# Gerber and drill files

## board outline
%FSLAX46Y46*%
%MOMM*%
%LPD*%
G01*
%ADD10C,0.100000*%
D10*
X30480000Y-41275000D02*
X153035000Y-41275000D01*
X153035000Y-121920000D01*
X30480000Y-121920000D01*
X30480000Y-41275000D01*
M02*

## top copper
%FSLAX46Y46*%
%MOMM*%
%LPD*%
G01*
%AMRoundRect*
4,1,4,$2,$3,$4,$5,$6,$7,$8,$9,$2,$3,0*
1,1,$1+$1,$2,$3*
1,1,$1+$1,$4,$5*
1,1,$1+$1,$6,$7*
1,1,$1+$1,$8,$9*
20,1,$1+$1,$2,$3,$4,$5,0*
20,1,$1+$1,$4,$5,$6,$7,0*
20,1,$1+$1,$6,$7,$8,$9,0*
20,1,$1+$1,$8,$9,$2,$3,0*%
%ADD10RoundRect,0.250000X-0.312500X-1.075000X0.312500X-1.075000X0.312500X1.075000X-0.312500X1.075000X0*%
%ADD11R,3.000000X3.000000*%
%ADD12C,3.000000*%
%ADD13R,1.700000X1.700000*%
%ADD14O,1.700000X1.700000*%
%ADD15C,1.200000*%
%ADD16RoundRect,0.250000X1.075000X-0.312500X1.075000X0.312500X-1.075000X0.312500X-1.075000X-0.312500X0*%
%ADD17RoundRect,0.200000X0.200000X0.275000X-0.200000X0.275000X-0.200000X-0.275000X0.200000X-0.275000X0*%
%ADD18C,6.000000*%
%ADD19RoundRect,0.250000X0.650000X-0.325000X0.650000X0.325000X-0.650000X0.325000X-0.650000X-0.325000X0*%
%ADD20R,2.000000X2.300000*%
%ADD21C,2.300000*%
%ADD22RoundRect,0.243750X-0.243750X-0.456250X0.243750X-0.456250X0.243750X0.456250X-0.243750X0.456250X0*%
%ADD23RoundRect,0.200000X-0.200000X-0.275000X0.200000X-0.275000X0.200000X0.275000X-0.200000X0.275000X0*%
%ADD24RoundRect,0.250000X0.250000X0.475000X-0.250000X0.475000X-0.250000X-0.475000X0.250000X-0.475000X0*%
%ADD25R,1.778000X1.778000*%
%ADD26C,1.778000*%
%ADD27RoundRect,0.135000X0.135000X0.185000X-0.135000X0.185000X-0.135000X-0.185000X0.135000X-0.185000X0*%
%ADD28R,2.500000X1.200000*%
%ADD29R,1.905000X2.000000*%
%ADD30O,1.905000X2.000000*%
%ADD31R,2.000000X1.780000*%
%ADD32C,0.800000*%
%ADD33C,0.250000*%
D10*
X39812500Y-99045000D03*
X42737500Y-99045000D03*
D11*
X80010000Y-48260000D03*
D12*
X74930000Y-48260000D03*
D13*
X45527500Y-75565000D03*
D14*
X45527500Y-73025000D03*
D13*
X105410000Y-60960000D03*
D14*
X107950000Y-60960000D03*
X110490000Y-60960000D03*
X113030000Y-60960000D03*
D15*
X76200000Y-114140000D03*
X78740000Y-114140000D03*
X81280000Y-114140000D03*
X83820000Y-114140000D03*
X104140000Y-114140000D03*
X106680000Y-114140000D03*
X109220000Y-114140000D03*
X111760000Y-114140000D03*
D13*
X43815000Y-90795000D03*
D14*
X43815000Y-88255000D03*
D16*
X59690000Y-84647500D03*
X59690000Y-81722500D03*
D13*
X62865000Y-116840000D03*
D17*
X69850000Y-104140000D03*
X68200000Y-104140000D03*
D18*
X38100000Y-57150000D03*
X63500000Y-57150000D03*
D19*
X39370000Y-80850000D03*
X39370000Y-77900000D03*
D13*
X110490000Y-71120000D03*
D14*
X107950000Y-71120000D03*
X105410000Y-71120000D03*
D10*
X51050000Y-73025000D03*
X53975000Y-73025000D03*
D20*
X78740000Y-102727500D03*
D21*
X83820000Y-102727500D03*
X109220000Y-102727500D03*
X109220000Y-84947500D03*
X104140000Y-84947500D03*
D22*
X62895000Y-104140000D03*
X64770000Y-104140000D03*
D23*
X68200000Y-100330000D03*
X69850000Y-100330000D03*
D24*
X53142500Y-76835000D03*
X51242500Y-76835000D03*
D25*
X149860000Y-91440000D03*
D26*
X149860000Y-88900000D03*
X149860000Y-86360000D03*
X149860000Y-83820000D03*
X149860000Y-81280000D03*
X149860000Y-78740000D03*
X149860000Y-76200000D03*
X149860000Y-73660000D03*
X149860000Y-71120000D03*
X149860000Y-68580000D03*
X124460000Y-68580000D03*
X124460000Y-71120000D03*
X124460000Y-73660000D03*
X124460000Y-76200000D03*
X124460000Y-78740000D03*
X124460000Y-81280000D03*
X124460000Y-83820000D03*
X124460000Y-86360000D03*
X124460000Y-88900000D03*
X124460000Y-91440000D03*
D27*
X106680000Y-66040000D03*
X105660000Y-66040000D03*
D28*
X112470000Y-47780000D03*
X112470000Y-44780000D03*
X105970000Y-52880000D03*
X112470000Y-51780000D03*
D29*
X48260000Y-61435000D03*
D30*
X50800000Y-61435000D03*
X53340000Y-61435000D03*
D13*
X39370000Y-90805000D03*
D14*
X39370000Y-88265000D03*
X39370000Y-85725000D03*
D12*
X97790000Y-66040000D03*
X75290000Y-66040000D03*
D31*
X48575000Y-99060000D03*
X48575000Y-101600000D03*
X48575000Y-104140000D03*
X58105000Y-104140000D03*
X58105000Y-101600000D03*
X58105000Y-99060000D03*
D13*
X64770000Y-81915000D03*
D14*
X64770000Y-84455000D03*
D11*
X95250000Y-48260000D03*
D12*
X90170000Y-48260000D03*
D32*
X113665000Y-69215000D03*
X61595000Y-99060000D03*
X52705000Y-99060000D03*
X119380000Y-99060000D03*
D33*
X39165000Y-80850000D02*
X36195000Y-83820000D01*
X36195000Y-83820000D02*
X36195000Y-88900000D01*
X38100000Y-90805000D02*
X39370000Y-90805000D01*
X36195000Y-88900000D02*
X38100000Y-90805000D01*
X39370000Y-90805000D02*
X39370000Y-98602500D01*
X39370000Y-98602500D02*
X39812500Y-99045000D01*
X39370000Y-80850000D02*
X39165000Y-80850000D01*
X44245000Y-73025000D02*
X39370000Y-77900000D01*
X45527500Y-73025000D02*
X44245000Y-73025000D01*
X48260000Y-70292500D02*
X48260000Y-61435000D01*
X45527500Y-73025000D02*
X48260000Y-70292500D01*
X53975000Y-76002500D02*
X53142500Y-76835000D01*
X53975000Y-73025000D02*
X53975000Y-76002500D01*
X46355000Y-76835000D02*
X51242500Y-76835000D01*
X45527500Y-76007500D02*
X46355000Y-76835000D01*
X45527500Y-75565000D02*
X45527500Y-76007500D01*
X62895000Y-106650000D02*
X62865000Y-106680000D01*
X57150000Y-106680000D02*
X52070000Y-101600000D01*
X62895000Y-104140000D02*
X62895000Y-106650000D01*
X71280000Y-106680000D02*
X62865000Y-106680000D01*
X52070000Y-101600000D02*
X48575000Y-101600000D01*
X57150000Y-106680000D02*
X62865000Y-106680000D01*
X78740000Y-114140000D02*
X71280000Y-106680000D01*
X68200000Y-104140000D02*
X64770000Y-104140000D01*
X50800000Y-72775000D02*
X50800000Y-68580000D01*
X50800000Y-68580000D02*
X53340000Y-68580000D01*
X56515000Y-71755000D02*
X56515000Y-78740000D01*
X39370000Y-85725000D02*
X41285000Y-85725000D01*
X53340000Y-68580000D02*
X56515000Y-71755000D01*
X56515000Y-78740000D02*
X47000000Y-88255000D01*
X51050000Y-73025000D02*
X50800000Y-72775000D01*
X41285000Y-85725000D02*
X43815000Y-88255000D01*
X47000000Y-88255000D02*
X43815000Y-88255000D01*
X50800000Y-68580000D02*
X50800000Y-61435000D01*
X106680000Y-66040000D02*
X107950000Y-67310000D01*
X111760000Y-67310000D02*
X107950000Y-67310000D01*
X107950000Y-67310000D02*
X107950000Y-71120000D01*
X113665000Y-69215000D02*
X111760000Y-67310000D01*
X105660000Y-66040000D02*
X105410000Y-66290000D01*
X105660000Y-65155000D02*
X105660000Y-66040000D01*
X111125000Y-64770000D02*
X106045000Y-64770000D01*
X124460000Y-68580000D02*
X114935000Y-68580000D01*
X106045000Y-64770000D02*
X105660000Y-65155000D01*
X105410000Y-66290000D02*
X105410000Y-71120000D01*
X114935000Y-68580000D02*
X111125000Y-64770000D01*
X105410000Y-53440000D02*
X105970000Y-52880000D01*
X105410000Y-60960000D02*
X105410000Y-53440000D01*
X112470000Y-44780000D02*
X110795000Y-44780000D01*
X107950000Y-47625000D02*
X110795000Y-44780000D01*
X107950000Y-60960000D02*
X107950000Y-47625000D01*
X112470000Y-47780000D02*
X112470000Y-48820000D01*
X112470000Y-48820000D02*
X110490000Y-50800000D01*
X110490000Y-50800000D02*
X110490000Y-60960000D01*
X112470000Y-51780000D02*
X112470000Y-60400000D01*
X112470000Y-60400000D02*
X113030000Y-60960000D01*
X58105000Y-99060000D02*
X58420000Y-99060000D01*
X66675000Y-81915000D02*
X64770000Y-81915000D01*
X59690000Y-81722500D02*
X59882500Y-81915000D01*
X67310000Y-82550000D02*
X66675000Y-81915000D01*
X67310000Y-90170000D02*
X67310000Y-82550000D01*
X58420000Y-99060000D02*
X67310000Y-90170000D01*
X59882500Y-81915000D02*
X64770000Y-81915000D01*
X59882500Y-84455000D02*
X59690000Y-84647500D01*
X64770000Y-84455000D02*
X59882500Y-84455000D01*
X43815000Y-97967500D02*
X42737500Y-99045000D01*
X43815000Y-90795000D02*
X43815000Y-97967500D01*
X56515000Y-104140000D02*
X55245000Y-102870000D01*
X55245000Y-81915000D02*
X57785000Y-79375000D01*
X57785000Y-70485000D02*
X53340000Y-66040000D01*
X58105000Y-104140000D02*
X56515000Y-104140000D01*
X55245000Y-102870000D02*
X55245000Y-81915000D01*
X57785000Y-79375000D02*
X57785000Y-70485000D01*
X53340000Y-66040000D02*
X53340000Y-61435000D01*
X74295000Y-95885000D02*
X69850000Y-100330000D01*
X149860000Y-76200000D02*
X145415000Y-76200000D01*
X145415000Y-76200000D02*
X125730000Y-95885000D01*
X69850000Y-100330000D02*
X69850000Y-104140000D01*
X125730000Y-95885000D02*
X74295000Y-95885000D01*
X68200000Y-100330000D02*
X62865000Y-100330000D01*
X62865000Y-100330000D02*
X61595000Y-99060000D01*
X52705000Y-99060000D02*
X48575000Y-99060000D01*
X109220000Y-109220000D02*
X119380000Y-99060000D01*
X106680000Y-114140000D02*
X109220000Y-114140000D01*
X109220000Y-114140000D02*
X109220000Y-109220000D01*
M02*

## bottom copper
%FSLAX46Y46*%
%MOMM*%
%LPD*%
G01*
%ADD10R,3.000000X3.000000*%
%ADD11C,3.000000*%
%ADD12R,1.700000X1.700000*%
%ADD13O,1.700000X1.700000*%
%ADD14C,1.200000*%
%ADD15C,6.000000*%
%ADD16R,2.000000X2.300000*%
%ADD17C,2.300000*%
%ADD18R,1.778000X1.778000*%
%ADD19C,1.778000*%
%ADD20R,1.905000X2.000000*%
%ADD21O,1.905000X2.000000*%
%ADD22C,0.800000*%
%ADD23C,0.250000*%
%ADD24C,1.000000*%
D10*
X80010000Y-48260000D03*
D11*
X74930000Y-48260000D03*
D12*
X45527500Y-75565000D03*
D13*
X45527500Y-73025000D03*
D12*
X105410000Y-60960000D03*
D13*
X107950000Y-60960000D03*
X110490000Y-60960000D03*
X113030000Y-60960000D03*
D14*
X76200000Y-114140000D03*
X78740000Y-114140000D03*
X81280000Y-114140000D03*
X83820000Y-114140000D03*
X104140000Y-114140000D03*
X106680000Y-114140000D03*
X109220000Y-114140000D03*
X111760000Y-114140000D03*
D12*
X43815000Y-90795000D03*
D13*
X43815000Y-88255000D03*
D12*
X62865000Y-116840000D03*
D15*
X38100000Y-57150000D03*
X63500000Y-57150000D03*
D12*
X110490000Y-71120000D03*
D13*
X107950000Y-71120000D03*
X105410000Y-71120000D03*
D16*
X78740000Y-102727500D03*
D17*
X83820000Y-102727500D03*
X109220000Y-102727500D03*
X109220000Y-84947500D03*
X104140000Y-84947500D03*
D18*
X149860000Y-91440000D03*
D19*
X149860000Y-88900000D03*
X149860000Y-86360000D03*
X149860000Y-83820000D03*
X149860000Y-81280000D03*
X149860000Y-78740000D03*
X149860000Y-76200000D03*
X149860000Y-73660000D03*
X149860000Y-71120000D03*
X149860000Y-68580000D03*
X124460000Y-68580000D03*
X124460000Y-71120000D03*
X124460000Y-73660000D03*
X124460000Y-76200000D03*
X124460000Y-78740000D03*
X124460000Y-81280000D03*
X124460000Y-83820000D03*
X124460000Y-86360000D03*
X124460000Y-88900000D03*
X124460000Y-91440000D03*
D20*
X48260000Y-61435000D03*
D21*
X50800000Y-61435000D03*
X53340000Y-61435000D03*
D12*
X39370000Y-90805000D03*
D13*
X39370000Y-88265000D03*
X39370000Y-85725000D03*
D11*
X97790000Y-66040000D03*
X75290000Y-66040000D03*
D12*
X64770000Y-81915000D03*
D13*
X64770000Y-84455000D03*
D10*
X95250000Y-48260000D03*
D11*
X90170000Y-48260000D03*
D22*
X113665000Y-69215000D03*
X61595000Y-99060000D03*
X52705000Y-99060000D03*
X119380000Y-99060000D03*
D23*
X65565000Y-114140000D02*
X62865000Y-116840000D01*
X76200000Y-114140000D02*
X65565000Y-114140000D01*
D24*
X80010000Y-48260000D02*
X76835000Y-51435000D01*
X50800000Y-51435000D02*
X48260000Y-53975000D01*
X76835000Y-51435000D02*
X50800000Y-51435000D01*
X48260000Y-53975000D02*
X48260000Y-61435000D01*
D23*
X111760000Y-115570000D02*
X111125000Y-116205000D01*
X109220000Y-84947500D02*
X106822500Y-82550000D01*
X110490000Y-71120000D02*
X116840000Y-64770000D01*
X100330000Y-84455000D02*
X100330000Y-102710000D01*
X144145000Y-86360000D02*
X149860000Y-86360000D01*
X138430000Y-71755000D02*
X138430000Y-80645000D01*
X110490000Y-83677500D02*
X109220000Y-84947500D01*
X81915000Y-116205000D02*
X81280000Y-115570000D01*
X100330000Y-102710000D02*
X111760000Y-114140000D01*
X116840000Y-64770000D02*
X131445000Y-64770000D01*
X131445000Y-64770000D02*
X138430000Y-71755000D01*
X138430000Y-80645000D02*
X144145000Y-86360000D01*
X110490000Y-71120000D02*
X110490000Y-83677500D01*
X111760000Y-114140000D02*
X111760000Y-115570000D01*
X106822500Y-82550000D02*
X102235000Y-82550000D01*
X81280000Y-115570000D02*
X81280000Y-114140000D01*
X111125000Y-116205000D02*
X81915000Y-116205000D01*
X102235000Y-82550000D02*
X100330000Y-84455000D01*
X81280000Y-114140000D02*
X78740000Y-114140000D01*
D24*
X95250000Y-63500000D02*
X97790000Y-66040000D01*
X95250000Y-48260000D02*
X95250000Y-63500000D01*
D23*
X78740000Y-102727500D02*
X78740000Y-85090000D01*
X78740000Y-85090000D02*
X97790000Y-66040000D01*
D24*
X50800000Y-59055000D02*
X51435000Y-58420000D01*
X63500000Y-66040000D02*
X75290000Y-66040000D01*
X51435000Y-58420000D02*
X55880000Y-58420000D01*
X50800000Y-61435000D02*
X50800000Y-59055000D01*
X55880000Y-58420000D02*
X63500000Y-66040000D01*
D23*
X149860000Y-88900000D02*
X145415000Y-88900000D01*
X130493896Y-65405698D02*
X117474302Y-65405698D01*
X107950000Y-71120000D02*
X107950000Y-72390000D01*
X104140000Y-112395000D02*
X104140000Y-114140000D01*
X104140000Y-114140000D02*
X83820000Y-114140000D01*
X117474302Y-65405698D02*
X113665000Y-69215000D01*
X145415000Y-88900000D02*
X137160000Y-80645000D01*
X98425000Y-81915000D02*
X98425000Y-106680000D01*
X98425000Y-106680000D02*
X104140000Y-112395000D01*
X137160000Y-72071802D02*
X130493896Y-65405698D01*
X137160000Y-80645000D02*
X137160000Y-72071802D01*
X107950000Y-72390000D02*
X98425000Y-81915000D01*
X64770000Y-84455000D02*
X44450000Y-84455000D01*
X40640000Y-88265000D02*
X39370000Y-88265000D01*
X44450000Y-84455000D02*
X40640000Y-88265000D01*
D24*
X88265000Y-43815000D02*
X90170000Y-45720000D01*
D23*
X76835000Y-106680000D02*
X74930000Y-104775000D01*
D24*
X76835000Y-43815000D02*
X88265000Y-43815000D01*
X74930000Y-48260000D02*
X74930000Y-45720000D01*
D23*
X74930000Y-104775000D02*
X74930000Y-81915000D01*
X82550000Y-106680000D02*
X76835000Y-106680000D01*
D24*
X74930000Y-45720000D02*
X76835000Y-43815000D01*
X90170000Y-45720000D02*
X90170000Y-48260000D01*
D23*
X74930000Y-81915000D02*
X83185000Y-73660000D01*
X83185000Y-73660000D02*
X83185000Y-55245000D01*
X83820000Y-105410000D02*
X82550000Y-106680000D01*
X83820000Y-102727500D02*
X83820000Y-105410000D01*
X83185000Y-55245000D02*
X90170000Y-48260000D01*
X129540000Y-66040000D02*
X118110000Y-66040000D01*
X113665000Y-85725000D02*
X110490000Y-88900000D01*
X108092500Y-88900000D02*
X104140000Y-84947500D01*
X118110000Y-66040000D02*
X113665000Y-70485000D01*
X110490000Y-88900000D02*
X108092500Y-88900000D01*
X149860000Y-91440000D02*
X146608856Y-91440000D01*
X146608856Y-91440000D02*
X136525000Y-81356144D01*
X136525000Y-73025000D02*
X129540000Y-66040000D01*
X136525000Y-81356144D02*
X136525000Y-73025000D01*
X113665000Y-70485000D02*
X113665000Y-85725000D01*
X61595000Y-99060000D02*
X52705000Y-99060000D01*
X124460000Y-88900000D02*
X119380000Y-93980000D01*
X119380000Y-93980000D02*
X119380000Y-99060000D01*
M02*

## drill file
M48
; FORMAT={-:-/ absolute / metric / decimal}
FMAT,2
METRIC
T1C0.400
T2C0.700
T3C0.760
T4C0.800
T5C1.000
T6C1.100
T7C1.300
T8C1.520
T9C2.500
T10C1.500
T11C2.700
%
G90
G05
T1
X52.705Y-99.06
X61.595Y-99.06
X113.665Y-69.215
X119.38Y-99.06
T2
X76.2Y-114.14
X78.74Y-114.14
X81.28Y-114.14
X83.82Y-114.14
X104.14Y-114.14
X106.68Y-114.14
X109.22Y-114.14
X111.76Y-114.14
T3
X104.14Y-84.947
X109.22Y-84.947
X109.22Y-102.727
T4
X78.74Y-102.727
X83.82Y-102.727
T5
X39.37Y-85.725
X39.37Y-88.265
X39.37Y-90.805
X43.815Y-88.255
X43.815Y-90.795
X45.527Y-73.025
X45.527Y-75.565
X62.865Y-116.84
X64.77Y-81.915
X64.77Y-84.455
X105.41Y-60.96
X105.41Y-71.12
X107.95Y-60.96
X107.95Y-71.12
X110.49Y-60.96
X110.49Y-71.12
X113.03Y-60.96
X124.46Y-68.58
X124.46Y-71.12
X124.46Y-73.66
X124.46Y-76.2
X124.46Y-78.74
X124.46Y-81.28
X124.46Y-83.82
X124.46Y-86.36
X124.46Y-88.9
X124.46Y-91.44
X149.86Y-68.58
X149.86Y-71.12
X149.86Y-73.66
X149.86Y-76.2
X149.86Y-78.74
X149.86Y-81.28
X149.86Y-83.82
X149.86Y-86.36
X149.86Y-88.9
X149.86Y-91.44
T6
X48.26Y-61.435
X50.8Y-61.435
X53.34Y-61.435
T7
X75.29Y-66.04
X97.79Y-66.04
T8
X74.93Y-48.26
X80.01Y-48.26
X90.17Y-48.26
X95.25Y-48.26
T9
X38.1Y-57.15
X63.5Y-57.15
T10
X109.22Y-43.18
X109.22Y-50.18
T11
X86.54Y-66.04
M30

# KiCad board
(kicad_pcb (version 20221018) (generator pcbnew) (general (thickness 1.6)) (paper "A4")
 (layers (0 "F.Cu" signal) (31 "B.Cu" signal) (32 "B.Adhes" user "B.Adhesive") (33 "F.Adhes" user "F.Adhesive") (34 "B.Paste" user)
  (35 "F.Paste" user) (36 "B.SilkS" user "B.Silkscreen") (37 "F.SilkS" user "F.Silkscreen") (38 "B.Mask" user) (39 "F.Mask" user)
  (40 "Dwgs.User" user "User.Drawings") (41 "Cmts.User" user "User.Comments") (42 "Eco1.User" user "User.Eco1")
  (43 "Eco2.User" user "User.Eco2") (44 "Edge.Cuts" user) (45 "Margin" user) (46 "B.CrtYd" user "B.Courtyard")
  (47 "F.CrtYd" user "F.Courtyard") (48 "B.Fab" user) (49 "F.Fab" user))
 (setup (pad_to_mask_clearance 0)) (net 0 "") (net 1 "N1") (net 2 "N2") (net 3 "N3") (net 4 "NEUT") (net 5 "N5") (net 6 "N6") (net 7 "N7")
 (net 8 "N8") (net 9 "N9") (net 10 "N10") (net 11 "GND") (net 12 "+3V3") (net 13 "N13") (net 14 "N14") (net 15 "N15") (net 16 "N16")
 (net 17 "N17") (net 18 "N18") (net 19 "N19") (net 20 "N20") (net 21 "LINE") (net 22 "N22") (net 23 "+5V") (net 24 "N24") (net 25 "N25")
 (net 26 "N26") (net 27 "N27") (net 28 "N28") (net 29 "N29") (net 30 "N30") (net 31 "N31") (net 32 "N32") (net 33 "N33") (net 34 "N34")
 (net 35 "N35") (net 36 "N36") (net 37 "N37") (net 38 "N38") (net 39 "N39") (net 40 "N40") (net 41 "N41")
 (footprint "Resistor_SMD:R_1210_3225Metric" (layer "F.Cu") (at 41.275 99.045)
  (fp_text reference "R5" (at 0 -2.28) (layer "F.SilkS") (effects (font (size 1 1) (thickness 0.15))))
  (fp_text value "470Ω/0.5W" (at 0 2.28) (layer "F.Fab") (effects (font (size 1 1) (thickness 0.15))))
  (pad "1" smd roundrect (at -1.4625 0) (size 1.125 2.65) (layers "F.Cu" "F.Paste" "F.Mask") (roundrect_rratio 0.2222222222) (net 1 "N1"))
  (pad "2" smd roundrect (at 1.4625 0) (size 1.125 2.65) (layers "F.Cu" "F.Paste" "F.Mask") (roundrect_rratio 0.2222222222) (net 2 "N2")))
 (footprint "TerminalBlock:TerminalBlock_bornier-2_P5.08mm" (layer "F.Cu") (at 80.01 48.26 180)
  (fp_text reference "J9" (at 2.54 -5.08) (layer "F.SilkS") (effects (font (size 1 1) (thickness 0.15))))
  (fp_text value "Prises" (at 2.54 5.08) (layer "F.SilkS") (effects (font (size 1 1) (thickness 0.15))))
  (pad "1" thru_hole rect (at 0 0 180) (size 3 3) (drill 1.52) (layers "*.Cu" "*.Mask") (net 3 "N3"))
  (pad "2" thru_hole circle (at 5.08 0 180) (size 3 3) (drill 1.52) (layers "*.Cu" "*.Mask") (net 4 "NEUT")))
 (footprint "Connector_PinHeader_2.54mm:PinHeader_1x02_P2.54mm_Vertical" (layer "F.Cu") (at 45.5275 75.565 180)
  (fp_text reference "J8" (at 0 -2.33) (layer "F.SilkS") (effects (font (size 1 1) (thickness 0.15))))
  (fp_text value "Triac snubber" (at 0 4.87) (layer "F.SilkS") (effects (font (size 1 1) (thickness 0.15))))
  (pad "1" thru_hole rect (at 0 0 180) (size 1.7 1.7) (drill 1) (layers "*.Cu" "*.Mask") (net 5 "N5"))
  (pad "2" thru_hole oval (at 0 2.54 180) (size 1.7 1.7) (drill 1) (layers "*.Cu" "*.Mask") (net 3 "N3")))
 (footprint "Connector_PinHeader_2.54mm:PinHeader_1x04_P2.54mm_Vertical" (layer "F.Cu") (at 105.41 60.96 90)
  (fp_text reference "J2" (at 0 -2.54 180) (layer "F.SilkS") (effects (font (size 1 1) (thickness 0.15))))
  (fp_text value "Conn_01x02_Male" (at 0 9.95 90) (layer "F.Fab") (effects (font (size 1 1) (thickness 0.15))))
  (pad "1" thru_hole rect (at 0 0 90) (size 1.7 1.7) (drill 1) (layers "*.Cu" "*.Mask") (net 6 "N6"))
  (pad "2" thru_hole oval (at 0 2.54 90) (size 1.7 1.7) (drill 1) (layers "*.Cu" "*.Mask") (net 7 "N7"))
  (pad "3" thru_hole oval (at 0 5.08 90) (size 1.7 1.7) (drill 1) (layers "*.Cu" "*.Mask") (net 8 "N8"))
  (pad "4" thru_hole oval (at 0 7.62 90) (size 1.7 1.7) (drill 1) (layers "*.Cu" "*.Mask") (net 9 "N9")))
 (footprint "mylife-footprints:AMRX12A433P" (layer "F.Cu") (at 93.98 116.84)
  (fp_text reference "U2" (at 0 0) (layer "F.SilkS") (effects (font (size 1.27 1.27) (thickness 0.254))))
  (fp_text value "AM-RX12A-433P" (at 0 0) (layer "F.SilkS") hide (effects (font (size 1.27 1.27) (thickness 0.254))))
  (pad "1" thru_hole circle (at -17.78 -2.7) (size 1.2 1.2) (drill 0.7) (layers "*.Cu" "*.Mask") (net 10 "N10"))
  (pad "2" thru_hole circle (at -15.24 -2.7) (size 1.2 1.2) (drill 0.7) (layers "*.Cu" "*.Mask") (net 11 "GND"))
  (pad "3" thru_hole circle (at -12.7 -2.7) (size 1.2 1.2) (drill 0.7) (layers "*.Cu" "*.Mask") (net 11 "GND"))
  (pad "4" thru_hole circle (at -10.16 -2.7) (size 1.2 1.2) (drill 0.7) (layers "*.Cu" "*.Mask") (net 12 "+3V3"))
  (pad "5" thru_hole circle (at 10.16 -2.7) (size 1.2 1.2) (drill 0.7) (layers "*.Cu" "*.Mask") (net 12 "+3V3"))
  (pad "6" thru_hole circle (at 12.7 -2.7) (size 1.2 1.2) (drill 0.7) (layers "*.Cu" "*.Mask") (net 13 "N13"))
  (pad "7" thru_hole circle (at 15.24 -2.7) (size 1.2 1.2) (drill 0.7) (layers "*.Cu" "*.Mask") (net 13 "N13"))
  (pad "8" thru_hole circle (at 17.78 -2.7) (size 1.2 1.2) (drill 0.7) (layers "*.Cu" "*.Mask") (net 11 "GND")))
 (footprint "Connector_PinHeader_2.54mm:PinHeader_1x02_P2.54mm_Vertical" (layer "F.Cu") (at 43.815 90.795 180)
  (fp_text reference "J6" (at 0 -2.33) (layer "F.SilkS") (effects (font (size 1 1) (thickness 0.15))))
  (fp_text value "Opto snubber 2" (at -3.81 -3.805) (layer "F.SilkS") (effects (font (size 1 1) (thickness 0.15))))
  (pad "1" thru_hole rect (at 0 0 180) (size 1.7 1.7) (drill 1) (layers "*.Cu" "*.Mask") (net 2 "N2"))
  (pad "2" thru_hole oval (at 0 2.54 180) (size 1.7 1.7) (drill 1) (layers "*.Cu" "*.Mask") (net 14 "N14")))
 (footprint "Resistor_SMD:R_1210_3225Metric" (layer "F.Cu") (at 59.69 83.185 90)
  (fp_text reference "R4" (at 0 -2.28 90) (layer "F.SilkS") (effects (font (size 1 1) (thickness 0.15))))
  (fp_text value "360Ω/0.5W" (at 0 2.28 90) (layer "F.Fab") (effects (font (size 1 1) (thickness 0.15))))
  (pad "1" smd roundrect (at -1.4625 0 90) (size 1.125 2.65) (layers "F.Cu" "F.Paste" "F.Mask") (roundrect_rratio 0.2222222222)
   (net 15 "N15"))
  (pad "2" smd roundrect (at 1.4625 0 90) (size 1.125 2.65) (layers "F.Cu" "F.Paste" "F.Mask") (roundrect_rratio 0.2222222222)
   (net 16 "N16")))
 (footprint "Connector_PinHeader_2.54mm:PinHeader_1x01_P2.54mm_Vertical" (layer "F.Cu") (at 62.865 116.84)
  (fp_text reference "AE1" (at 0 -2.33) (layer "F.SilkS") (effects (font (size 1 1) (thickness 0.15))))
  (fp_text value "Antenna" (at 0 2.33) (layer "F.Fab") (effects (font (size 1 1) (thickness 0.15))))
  (pad "1" thru_hole rect (at 0 0) (size 1.7 1.7) (drill 1) (layers "*.Cu" "*.Mask") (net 10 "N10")))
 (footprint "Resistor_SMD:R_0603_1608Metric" (layer "F.Cu") (at 69.025 104.14 180)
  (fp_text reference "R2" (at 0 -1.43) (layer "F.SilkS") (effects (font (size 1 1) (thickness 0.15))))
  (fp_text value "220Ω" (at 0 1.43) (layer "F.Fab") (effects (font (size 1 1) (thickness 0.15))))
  (pad "1" smd roundrect (at -0.825 0 180) (size 0.8 0.95) (layers "F.Cu" "F.Paste" "F.Mask") (roundrect_rratio 0.25) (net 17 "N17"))
  (pad "2" smd roundrect (at 0.825 0 180) (size 0.8 0.95) (layers "F.Cu" "F.Paste" "F.Mask") (roundrect_rratio 0.25) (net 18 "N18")))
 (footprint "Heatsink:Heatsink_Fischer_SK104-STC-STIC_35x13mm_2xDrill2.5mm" (layer "F.Cu") (at 50.8 57.15)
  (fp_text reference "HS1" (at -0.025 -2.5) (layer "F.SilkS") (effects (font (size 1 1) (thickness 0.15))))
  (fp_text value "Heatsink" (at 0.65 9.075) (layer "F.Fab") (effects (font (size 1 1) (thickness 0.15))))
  (pad "1" thru_hole circle (at -12.7 0 180) (size 6 6) (drill 2.5) (layers "*.Cu" "*.Mask"))
  (pad "1" thru_hole circle (at 12.7 0) (size 6 6) (drill 2.5) (layers "*.Cu" "*.Mask")))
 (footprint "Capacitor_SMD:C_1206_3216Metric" (layer "F.Cu") (at 39.37 79.375 90)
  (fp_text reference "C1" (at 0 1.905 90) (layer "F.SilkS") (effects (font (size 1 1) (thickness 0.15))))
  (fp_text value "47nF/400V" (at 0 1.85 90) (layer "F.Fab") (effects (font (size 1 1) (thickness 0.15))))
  (pad "1" smd roundrect (at -1.475 0 90) (size 1.15 1.8) (layers "F.Cu" "F.Paste" "F.Mask") (roundrect_rratio 0.2173913043) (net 1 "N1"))
  (pad "2" smd roundrect (at 1.475 0 90) (size 1.15 1.8) (layers "F.Cu" "F.Paste" "F.Mask") (roundrect_rratio 0.2173913043) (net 3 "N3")))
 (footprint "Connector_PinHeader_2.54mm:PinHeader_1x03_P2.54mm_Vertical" (layer "F.Cu") (at 110.49 71.12 -90)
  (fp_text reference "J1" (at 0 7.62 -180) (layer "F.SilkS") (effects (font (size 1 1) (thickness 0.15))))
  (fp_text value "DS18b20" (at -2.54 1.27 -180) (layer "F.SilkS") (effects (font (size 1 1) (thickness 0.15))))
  (pad "1" thru_hole rect (at 0 0 270) (size 1.7 1.7) (drill 1) (layers "*.Cu" "*.Mask") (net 11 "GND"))
  (pad "2" thru_hole oval (at 0 2.54 270) (size 1.7 1.7) (drill 1) (layers "*.Cu" "*.Mask") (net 12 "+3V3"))
  (pad "3" thru_hole oval (at 0 5.08 270) (size 1.7 1.7) (drill 1) (layers "*.Cu" "*.Mask") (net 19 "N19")))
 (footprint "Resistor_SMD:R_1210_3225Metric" (layer "F.Cu") (at 52.5125 73.025)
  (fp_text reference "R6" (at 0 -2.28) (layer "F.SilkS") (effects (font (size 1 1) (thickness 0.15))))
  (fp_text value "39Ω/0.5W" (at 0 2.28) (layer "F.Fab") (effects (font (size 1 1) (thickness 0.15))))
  (pad "1" smd roundrect (at -1.4625 0) (size 1.125 2.65) (layers "F.Cu" "F.Paste" "F.Mask") (roundrect_rratio 0.2222222222) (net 14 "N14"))
  (pad "2" smd roundrect (at 1.4625 0) (size 1.125 2.65) (layers "F.Cu" "F.Paste" "F.Mask") (roundrect_rratio 0.2222222222) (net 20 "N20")))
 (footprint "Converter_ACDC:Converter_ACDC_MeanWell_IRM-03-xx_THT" (layer "F.Cu") (at 78.74 102.7275 90)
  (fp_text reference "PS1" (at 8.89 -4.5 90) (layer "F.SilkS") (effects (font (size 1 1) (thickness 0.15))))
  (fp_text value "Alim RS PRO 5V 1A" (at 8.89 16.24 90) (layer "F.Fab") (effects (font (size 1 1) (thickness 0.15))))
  (pad "1" thru_hole rect (at 0 0 90) (size 2.3 2) (drill 0.8) (layers "*.Cu" "*.Mask") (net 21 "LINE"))
  (pad "3" thru_hole circle (at 0 5.08 90) (size 2.3 2.3) (drill 0.8) (layers "*.Cu" "*.Mask") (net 4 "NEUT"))
  (pad "5" thru_hole circle (at 0 30.48 90) (size 2.3 2.3) (drill 0.76) (layers "*.Cu" "*.Mask") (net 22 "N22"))
  (pad "14" thru_hole circle (at 17.78 30.48 90) (size 2.3 2.3) (drill 0.76) (layers "*.Cu" "*.Mask") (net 11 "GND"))
  (pad "16" thru_hole circle (at 17.78 25.4 90) (size 2.3 2.3) (drill 0.76) (layers "*.Cu" "*.Mask") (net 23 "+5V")))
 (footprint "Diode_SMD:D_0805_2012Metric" (layer "F.Cu") (at 63.8325 104.14)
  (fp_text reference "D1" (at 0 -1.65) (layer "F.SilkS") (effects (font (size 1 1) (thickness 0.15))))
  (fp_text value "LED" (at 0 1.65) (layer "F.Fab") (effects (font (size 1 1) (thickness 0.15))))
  (pad "1" smd roundrect (at -0.9375 0) (size 0.975 1.4) (layers "F.Cu" "F.Paste" "F.Mask") (roundrect_rratio 0.25) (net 11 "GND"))
  (pad "2" smd roundrect (at 0.9375 0) (size 0.975 1.4) (layers "F.Cu" "F.Paste" "F.Mask") (roundrect_rratio 0.25) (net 18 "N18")))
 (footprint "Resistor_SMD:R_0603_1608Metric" (layer "F.Cu") (at 69.025 100.33)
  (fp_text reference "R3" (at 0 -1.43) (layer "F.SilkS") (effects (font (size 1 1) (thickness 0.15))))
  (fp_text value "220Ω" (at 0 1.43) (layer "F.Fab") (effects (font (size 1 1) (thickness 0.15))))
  (pad "1" smd roundrect (at -0.825 0) (size 0.8 0.95) (layers "F.Cu" "F.Paste" "F.Mask") (roundrect_rratio 0.25) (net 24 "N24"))
  (pad "2" smd roundrect (at 0.825 0) (size 0.8 0.95) (layers "F.Cu" "F.Paste" "F.Mask") (roundrect_rratio 0.25) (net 17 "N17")))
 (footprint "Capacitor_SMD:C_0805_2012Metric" (layer "F.Cu") (at 52.1925 76.835 180)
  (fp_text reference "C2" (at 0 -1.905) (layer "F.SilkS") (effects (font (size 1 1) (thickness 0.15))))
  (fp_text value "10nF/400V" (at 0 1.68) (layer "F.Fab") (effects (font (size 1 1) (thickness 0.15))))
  (pad "1" smd roundrect (at -0.95 0 180) (size 1 1.45) (layers "F.Cu" "F.Paste" "F.Mask") (roundrect_rratio 0.25) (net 20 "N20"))
  (pad "2" smd roundrect (at 0.95 0 180) (size 1 1.45) (layers "F.Cu" "F.Paste" "F.Mask") (roundrect_rratio 0.25) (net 5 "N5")))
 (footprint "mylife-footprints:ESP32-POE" (layer "F.Cu") (at 137.12 81.41 180)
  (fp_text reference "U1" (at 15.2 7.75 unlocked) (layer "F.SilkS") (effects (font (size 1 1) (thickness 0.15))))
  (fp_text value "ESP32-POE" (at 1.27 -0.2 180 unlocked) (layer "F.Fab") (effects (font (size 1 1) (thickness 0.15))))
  (pad "1" thru_hole rect (at -12.74 -10.03 90) (size 1.778 1.778) (drill 1) (layers "*.Cu" "*.Mask") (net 23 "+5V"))
  (pad "2" thru_hole circle (at -12.74 -7.49 90) (size 1.778 1.778) (drill 1) (layers "*.Cu" "*.Mask") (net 12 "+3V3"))
  (pad "3" thru_hole circle (at -12.74 -4.95 90) (size 1.778 1.778) (drill 1) (layers "*.Cu" "*.Mask") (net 11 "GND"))
  (pad "4" thru_hole circle (at -12.74 -2.41 90) (size 1.778 1.778) (drill 1) (layers "*.Cu" "*.Mask") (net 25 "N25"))
  (pad "5" thru_hole circle (at -12.74 0.13 90) (size 1.778 1.778) (drill 1) (layers "*.Cu" "*.Mask") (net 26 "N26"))
  (pad "6" thru_hole circle (at -12.74 2.67 90) (size 1.778 1.778) (drill 1) (layers "*.Cu" "*.Mask") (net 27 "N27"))
  (pad "7" thru_hole circle (at -12.74 5.21 90) (size 1.778 1.778) (drill 1) (layers "*.Cu" "*.Mask") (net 17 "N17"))
  (pad "8" thru_hole circle (at -12.74 7.75 90) (size 1.778 1.778) (drill 1) (layers "*.Cu" "*.Mask") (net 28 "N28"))
  (pad "9" thru_hole circle (at -12.74 10.29 90) (size 1.778 1.778) (drill 1) (layers "*.Cu" "*.Mask") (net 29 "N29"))
  (pad "10" thru_hole circle (at -12.74 12.83 90) (size 1.778 1.778) (drill 1) (layers "*.Cu" "*.Mask") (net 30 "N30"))
  (pad "11" thru_hole circle (at 12.66 12.83 90) (size 1.778 1.778) (drill 1) (layers "*.Cu" "*.Mask") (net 19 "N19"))
  (pad "12" thru_hole circle (at 12.66 10.29 90) (size 1.778 1.778) (drill 1) (layers "*.Cu" "*.Mask") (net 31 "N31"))
  (pad "13" thru_hole circle (at 12.66 7.75 90) (size 1.778 1.778) (drill 1) (layers "*.Cu" "*.Mask") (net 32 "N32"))
  (pad "14" thru_hole circle (at 12.66 5.21 90) (size 1.778 1.778) (drill 1) (layers "*.Cu" "*.Mask") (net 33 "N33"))
  (pad "15" thru_hole circle (at 12.66 2.67 90) (size 1.778 1.778) (drill 1) (layers "*.Cu" "*.Mask") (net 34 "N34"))
  (pad "16" thru_hole circle (at 12.66 0.13 90) (size 1.778 1.778) (drill 1) (layers "*.Cu" "*.Mask") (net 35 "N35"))
  (pad "17" thru_hole circle (at 12.66 -2.41 90) (size 1.778 1.778) (drill 1) (layers "*.Cu" "*.Mask") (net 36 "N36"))
  (pad "18" thru_hole circle (at 12.66 -4.95 90) (size 1.778 1.778) (drill 1) (layers "*.Cu" "*.Mask") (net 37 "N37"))
  (pad "19" thru_hole circle (at 12.66 -7.49 90) (size 1.778 1.778) (drill 1) (layers "*.Cu" "*.Mask") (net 13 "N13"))
  (pad "20" thru_hole circle (at 12.66 -10.03 90) (size 1.778 1.778) (drill 1) (layers "*.Cu" "*.Mask") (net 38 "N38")))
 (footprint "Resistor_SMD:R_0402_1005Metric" (layer "F.Cu") (at 106.17 66.04 180)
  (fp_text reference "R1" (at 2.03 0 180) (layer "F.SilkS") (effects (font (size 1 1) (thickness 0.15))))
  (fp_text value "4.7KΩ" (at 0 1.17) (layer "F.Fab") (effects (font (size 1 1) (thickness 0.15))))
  (pad "1" smd roundrect (at -0.51 0 180) (size 0.54 0.64) (layers "F.Cu" "F.Paste" "F.Mask") (roundrect_rratio 0.25) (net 12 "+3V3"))
  (pad "2" smd roundrect (at 0.51 0 180) (size 0.54 0.64) (layers "F.Cu" "F.Paste" "F.Mask") (roundrect_rratio 0.25) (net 19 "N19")))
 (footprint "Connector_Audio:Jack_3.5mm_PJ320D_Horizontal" (layer "F.Cu") (at 109.22 47.955 -90)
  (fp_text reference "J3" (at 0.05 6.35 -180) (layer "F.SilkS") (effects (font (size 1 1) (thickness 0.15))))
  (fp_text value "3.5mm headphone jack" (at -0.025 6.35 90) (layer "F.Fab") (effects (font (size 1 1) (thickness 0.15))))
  (pad "" np_thru_hole circle (at -4.775 0 270) (size 1.5 1.5) (drill 1.5) (layers "*.Cu" "*.Mask"))
  (pad "" np_thru_hole circle (at 2.225 0 270) (size 1.5 1.5) (drill 1.5) (layers "*.Cu" "*.Mask"))
  (pad "R1" smd rect (at -0.175 -3.25 270) (size 1.2 2.5) (layers "F.Cu" "F.Paste" "F.Mask") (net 8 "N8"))
  (pad "R2" smd rect (at -3.175 -3.25 270) (size 1.2 2.5) (layers "F.Cu" "F.Paste" "F.Mask") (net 7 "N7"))
  (pad "S" smd rect (at 4.925 3.25 270) (size 1.2 2.5) (layers "F.Cu" "F.Paste" "F.Mask") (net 6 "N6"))
  (pad "T" smd rect (at 3.825 -3.25 270) (size 1.2 2.5) (layers "F.Cu" "F.Paste" "F.Mask") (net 9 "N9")))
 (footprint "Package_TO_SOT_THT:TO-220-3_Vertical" (layer "F.Cu") (at 48.26 61.435)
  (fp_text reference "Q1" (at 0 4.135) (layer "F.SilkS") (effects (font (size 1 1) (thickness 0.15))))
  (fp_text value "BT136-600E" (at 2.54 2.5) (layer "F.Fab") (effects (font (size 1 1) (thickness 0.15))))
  (pad "1" thru_hole rect (at 0 0) (size 1.905 2) (drill 1.1) (layers "*.Cu" "*.Mask") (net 3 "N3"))
  (pad "2" thru_hole oval (at 2.54 0) (size 1.905 2) (drill 1.1) (layers "*.Cu" "*.Mask") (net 14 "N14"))
  (pad "3" thru_hole oval (at 5.08 0) (size 1.905 2) (drill 1.1) (layers "*.Cu" "*.Mask") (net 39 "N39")))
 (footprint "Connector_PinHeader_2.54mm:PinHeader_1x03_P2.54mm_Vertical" (layer "F.Cu") (at 39.37 90.805 180)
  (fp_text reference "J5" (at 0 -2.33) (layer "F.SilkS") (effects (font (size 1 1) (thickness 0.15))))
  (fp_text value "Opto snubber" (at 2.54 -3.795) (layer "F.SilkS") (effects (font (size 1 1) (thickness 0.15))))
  (pad "1" thru_hole rect (at 0 0 180) (size 1.7 1.7) (drill 1) (layers "*.Cu" "*.Mask") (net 1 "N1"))
  (pad "2" thru_hole oval (at 0 2.54 180) (size 1.7 1.7) (drill 1) (layers "*.Cu" "*.Mask") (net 15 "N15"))
  (pad "3" thru_hole oval (at 0 5.08 180) (size 1.7 1.7) (drill 1) (layers "*.Cu" "*.Mask") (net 14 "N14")))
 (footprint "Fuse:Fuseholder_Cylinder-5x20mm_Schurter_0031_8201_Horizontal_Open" (layer "F.Cu") (at 97.79 66.04 180)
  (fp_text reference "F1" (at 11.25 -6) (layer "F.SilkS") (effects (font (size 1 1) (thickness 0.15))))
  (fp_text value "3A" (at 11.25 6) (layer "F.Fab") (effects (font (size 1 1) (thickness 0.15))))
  (pad "" np_thru_hole circle (at 11.25 0 180) (size 2.7 2.7) (drill 2.7) (layers "*.Cu" "*.Mask"))
  (pad "1" thru_hole circle (at 0 0 180) (size 3 3) (drill 1.3) (layers "*.Cu" "*.Mask") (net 21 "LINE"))
  (pad "2" thru_hole circle (at 22.5 0 180) (size 3 3) (drill 1.3) (layers "*.Cu" "*.Mask") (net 14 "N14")))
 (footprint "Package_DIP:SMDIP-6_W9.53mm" (layer "F.Cu") (at 53.34 101.6)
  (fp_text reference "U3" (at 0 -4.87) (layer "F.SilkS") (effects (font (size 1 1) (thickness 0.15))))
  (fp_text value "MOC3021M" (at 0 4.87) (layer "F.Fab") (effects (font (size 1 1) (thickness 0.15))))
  (pad "1" smd rect (at -4.765 -2.54) (size 2 1.78) (layers "F.Cu" "F.Paste" "F.Mask") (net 24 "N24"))
  (pad "2" smd rect (at -4.765 0) (size 2 1.78) (layers "F.Cu" "F.Paste" "F.Mask") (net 11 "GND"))
  (pad "3" smd rect (at -4.765 2.54) (size 2 1.78) (layers "F.Cu" "F.Paste" "F.Mask") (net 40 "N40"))
  (pad "4" smd rect (at 4.765 2.54) (size 2 1.78) (layers "F.Cu" "F.Paste" "F.Mask") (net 39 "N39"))
  (pad "5" smd rect (at 4.765 0) (size 2 1.78) (layers "F.Cu" "F.Paste" "F.Mask") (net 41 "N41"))
  (pad "6" smd rect (at 4.765 -2.54) (size 2 1.78) (layers "F.Cu" "F.Paste" "F.Mask") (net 16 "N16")))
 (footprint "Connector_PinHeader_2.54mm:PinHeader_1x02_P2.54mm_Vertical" (layer "F.Cu") (at 64.77 81.915)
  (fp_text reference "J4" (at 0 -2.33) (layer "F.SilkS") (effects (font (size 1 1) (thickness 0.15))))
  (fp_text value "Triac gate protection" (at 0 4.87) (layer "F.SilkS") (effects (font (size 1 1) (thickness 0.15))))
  (pad "1" thru_hole rect (at 0 0) (size 1.7 1.7) (drill 1) (layers "*.Cu" "*.Mask") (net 16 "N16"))
  (pad "2" thru_hole oval (at 0 2.54) (size 1.7 1.7) (drill 1) (layers "*.Cu" "*.Mask") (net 15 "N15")))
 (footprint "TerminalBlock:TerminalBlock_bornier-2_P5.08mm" (layer "F.Cu") (at 95.25 48.26 180)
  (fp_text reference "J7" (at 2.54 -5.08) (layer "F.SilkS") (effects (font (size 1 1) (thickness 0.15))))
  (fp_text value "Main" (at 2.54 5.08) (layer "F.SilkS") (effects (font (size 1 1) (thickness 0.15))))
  (pad "1" thru_hole rect (at 0 0 180) (size 3 3) (drill 1.52) (layers "*.Cu" "*.Mask") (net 21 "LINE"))
  (pad "2" thru_hole circle (at 5.08 0 180) (size 3 3) (drill 1.52) (layers "*.Cu" "*.Mask") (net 4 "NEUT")))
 (gr_rect (start 30.48 41.275) (end 153.035 121.92) (stroke (width 0.1) (type default)) (fill none) (layer "Edge.Cuts"))
 (segment (start 65.565 114.14) (end 62.865 116.84) (width 0.25) (layer "B.Cu") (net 10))
 (segment (start 76.2 114.14) (end 65.565 114.14) (width 0.25) (layer "B.Cu") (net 10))
 (segment (start 39.165 80.85) (end 36.195 83.82) (width 0.25) (layer "F.Cu") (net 1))
 (segment (start 36.195 83.82) (end 36.195 88.9) (width 0.25) (layer "F.Cu") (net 1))
 (segment (start 38.1 90.805) (end 39.37 90.805) (width 0.25) (layer "F.Cu") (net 1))
 (segment (start 36.195 88.9) (end 38.1 90.805) (width 0.25) (layer "F.Cu") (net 1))
 (segment (start 39.37 90.805) (end 39.37 98.6025) (width 0.25) (layer "F.Cu") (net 1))
 (segment (start 39.37 98.6025) (end 39.8125 99.045) (width 0.25) (layer "F.Cu") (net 1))
 (segment (start 39.37 80.85) (end 39.165 80.85) (width 0.25) (layer "F.Cu") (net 1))
 (segment (start 44.245 73.025) (end 39.37 77.9) (width 0.25) (layer "F.Cu") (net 3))
 (segment (start 45.5275 73.025) (end 44.245 73.025) (width 0.25) (layer "F.Cu") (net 3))
 (segment (start 48.26 70.2925) (end 48.26 61.435) (width 0.25) (layer "F.Cu") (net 3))
 (segment (start 45.5275 73.025) (end 48.26 70.2925) (width 0.25) (layer "F.Cu") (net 3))
 (segment (start 80.01 48.26) (end 76.835 51.435) (width 1) (layer "B.Cu") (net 3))
 (segment (start 50.8 51.435) (end 48.26 53.975) (width 1) (layer "B.Cu") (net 3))
 (segment (start 76.835 51.435) (end 50.8 51.435) (width 1) (layer "B.Cu") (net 3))
 (segment (start 48.26 53.975) (end 48.26 61.435) (width 1) (layer "B.Cu") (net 3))
 (segment (start 53.975 76.0025) (end 53.1425 76.835) (width 0.25) (layer "F.Cu") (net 20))
 (segment (start 53.975 73.025) (end 53.975 76.0025) (width 0.25) (layer "F.Cu") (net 20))
 (segment (start 46.355 76.835) (end 51.2425 76.835) (width 0.25) (layer "F.Cu") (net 5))
 (segment (start 45.5275 76.0075) (end 46.355 76.835) (width 0.25) (layer "F.Cu") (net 5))
 (segment (start 45.5275 75.565) (end 45.5275 76.0075) (width 0.25) (layer "F.Cu") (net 5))
 (segment (start 62.895 106.65) (end 62.865 106.68) (width 0.25) (layer "F.Cu") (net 11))
 (segment (start 57.15 106.68) (end 52.07 101.6) (width 0.25) (layer "F.Cu") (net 11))
 (segment (start 62.895 104.14) (end 62.895 106.65) (width 0.25) (layer "F.Cu") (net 11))
 (segment (start 71.28 106.68) (end 62.865 106.68) (width 0.25) (layer "F.Cu") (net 11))
 (segment (start 52.07 101.6) (end 48.575 101.6) (width 0.25) (layer "F.Cu") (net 11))
 (segment (start 57.15 106.68) (end 62.865 106.68) (width 0.25) (layer "F.Cu") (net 11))
 (segment (start 78.74 114.14) (end 71.28 106.68) (width 0.25) (layer "F.Cu") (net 11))
 (segment (start 111.76 115.57) (end 111.125 116.205) (width 0.25) (layer "B.Cu") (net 11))
 (segment (start 109.22 84.9475) (end 106.8225 82.55) (width 0.25) (layer "B.Cu") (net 11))
 (segment (start 110.49 71.12) (end 116.84 64.77) (width 0.25) (layer "B.Cu") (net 11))
 (segment (start 100.33 84.455) (end 100.33 102.71) (width 0.25) (layer "B.Cu") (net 11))
 (segment (start 144.145 86.36) (end 149.86 86.36) (width 0.25) (layer "B.Cu") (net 11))
 (segment (start 138.43 71.755) (end 138.43 80.645) (width 0.25) (layer "B.Cu") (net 11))
 (segment (start 110.49 83.6775) (end 109.22 84.9475) (width 0.25) (layer "B.Cu") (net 11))
 (segment (start 81.915 116.205) (end 81.28 115.57) (width 0.25) (layer "B.Cu") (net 11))
 (segment (start 100.33 102.71) (end 111.76 114.14) (width 0.25) (layer "B.Cu") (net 11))
 (segment (start 116.84 64.77) (end 131.445 64.77) (width 0.25) (layer "B.Cu") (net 11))
 (segment (start 131.445 64.77) (end 138.43 71.755) (width 0.25) (layer "B.Cu") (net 11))
 (segment (start 138.43 80.645) (end 144.145 86.36) (width 0.25) (layer "B.Cu") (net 11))
 (segment (start 110.49 71.12) (end 110.49 83.6775) (width 0.25) (layer "B.Cu") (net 11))
 (segment (start 111.76 114.14) (end 111.76 115.57) (width 0.25) (layer "B.Cu") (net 11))
 (segment (start 106.8225 82.55) (end 102.235 82.55) (width 0.25) (layer "B.Cu") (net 11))
 (segment (start 81.28 115.57) (end 81.28 114.14) (width 0.25) (layer "B.Cu") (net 11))
 (segment (start 111.125 116.205) (end 81.915 116.205) (width 0.25) (layer "B.Cu") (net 11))
 (segment (start 102.235 82.55) (end 100.33 84.455) (width 0.25) (layer "B.Cu") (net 11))
 (segment (start 81.28 114.14) (end 78.74 114.14) (width 0.25) (layer "B.Cu") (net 11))
 (segment (start 68.2 104.14) (end 64.77 104.14) (width 0.25) (layer "F.Cu") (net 18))
 (segment (start 95.25 63.5) (end 97.79 66.04) (width 1) (layer "B.Cu") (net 21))
 (segment (start 95.25 48.26) (end 95.25 63.5) (width 1) (layer "B.Cu") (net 21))
 (segment (start 78.74 102.7275) (end 78.74 85.09) (width 0.25) (layer "B.Cu") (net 21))
 (segment (start 78.74 85.09) (end 97.79 66.04) (width 0.25) (layer "B.Cu") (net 21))
 (segment (start 50.8 72.775) (end 50.8 68.58) (width 0.25) (layer "F.Cu") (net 14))
 (segment (start 50.8 68.58) (end 53.34 68.58) (width 0.25) (layer "F.Cu") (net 14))
 (segment (start 56.515 71.755) (end 56.515 78.74) (width 0.25) (layer "F.Cu") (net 14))
 (segment (start 39.37 85.725) (end 41.285 85.725) (width 0.25) (layer "F.Cu") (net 14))
 (segment (start 53.34 68.58) (end 56.515 71.755) (width 0.25) (layer "F.Cu") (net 14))
 (segment (start 56.515 78.74) (end 47 88.255) (width 0.25) (layer "F.Cu") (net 14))
 (segment (start 51.05 73.025) (end 50.8 72.775) (width 0.25) (layer "F.Cu") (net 14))
 (segment (start 41.285 85.725) (end 43.815 88.255) (width 0.25) (layer "F.Cu") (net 14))
 (segment (start 47 88.255) (end 43.815 88.255) (width 0.25) (layer "F.Cu") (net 14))
 (segment (start 50.8 68.58) (end 50.8 61.435) (width 0.25) (layer "F.Cu") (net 14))
 (segment (start 50.8 59.055) (end 51.435 58.42) (width 1) (layer "B.Cu") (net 14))
 (segment (start 63.5 66.04) (end 75.29 66.04) (width 1) (layer "B.Cu") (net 14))
 (segment (start 51.435 58.42) (end 55.88 58.42) (width 1) (layer "B.Cu") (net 14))
 (segment (start 50.8 61.435) (end 50.8 59.055) (width 1) (layer "B.Cu") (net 14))
 (segment (start 55.88 58.42) (end 63.5 66.04) (width 1) (layer "B.Cu") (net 14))
 (segment (start 106.68 66.04) (end 107.95 67.31) (width 0.25) (layer "F.Cu") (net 12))
 (segment (start 111.76 67.31) (end 107.95 67.31) (width 0.25) (layer "F.Cu") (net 12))
 (segment (start 107.95 67.31) (end 107.95 71.12) (width 0.25) (layer "F.Cu") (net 12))
 (segment (start 113.665 69.215) (end 111.76 67.31) (width 0.25) (layer "F.Cu") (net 12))
 (via (at 113.665 69.215) (size 0.8) (drill 0.4) (layers "F.Cu" "B.Cu") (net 12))
 (segment (start 149.86 88.9) (end 145.415 88.9) (width 0.25) (layer "B.Cu") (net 12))
 (segment (start 130.493896 65.405698) (end 117.474302 65.405698) (width 0.25) (layer "B.Cu") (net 12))
 (segment (start 107.95 71.12) (end 107.95 72.39) (width 0.25) (layer "B.Cu") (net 12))
 (segment (start 104.14 112.395) (end 104.14 114.14) (width 0.25) (layer "B.Cu") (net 12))
 (segment (start 104.14 114.14) (end 83.82 114.14) (width 0.25) (layer "B.Cu") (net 12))
 (segment (start 117.474302 65.405698) (end 113.665 69.215) (width 0.25) (layer "B.Cu") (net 12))
 (segment (start 145.415 88.9) (end 137.16 80.645) (width 0.25) (layer "B.Cu") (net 12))
 (segment (start 98.425 81.915) (end 98.425 106.68) (width 0.25) (layer "B.Cu") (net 12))
 (segment (start 98.425 106.68) (end 104.14 112.395) (width 0.25) (layer "B.Cu") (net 12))
 (segment (start 137.16 72.071802) (end 130.493896 65.405698) (width 0.25) (layer "B.Cu") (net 12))
 (segment (start 137.16 80.645) (end 137.16 72.071802) (width 0.25) (layer "B.Cu") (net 12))
 (segment (start 107.95 72.39) (end 98.425 81.915) (width 0.25) (layer "B.Cu") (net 12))
 (segment (start 105.66 66.04) (end 105.41 66.29) (width 0.25) (layer "F.Cu") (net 19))
 (segment (start 105.66 65.155) (end 105.66 66.04) (width 0.25) (layer "F.Cu") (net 19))
 (segment (start 111.125 64.77) (end 106.045 64.77) (width 0.25) (layer "F.Cu") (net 19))
 (segment (start 124.46 68.58) (end 114.935 68.58) (width 0.25) (layer "F.Cu") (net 19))
 (segment (start 106.045 64.77) (end 105.66 65.155) (width 0.25) (layer "F.Cu") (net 19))
 (segment (start 105.41 66.29) (end 105.41 71.12) (width 0.25) (layer "F.Cu") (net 19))
 (segment (start 114.935 68.58) (end 111.125 64.77) (width 0.25) (layer "F.Cu") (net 19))
 (segment (start 105.41 53.44) (end 105.97 52.88) (width 0.25) (layer "F.Cu") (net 6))
 (segment (start 105.41 60.96) (end 105.41 53.44) (width 0.25) (layer "F.Cu") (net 6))
 (segment (start 112.47 44.78) (end 110.795 44.78) (width 0.25) (layer "F.Cu") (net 7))
 (segment (start 107.95 47.625) (end 110.795 44.78) (width 0.25) (layer "F.Cu") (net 7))
 (segment (start 107.95 60.96) (end 107.95 47.625) (width 0.25) (layer "F.Cu") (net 7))
 (segment (start 112.47 47.78) (end 112.47 48.82) (width 0.25) (layer "F.Cu") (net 8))
 (segment (start 112.47 48.82) (end 110.49 50.8) (width 0.25) (layer "F.Cu") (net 8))
 (segment (start 110.49 50.8) (end 110.49 60.96) (width 0.25) (layer "F.Cu") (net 8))
 (segment (start 112.47 51.78) (end 112.47 60.4) (width 0.25) (layer "F.Cu") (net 9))
 (segment (start 112.47 60.4) (end 113.03 60.96) (width 0.25) (layer "F.Cu") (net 9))
 (segment (start 58.105 99.06) (end 58.42 99.06) (width 0.25) (layer "F.Cu") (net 16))
 (segment (start 66.675 81.915) (end 64.77 81.915) (width 0.25) (layer "F.Cu") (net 16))
 (segment (start 59.69 81.7225) (end 59.8825 81.915) (width 0.25) (layer "F.Cu") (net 16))
 (segment (start 67.31 82.55) (end 66.675 81.915) (width 0.25) (layer "F.Cu") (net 16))
 (segment (start 67.31 90.17) (end 67.31 82.55) (width 0.25) (layer "F.Cu") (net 16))
 (segment (start 58.42 99.06) (end 67.31 90.17) (width 0.25) (layer "F.Cu") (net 16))
 (segment (start 59.8825 81.915) (end 64.77 81.915) (width 0.25) (layer "F.Cu") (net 16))
 (segment (start 59.8825 84.455) (end 59.69 84.6475) (width 0.25) (layer "F.Cu") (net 15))
 (segment (start 64.77 84.455) (end 59.8825 84.455) (width 0.25) (layer "F.Cu") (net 15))
 (segment (start 64.77 84.455) (end 44.45 84.455) (width 0.25) (layer "B.Cu") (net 15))
 (segment (start 40.64 88.265) (end 39.37 88.265) (width 0.25) (layer "B.Cu") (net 15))
 (segment (start 44.45 84.455) (end 40.64 88.265) (width 0.25) (layer "B.Cu") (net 15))
 (segment (start 43.815 97.9675) (end 42.7375 99.045) (width 0.25) (layer "F.Cu") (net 2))
 (segment (start 43.815 90.795) (end 43.815 97.9675) (width 0.25) (layer "F.Cu") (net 2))
 (segment (start 88.265 43.815) (end 90.17 45.72) (width 1) (layer "B.Cu") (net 4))
 (segment (start 76.835 106.68) (end 74.93 104.775) (width 0.25) (layer "B.Cu") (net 4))
 (segment (start 76.835 43.815) (end 88.265 43.815) (width 1) (layer "B.Cu") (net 4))
 (segment (start 74.93 48.26) (end 74.93 45.72) (width 1) (layer "B.Cu") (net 4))
 (segment (start 74.93 104.775) (end 74.93 81.915) (width 0.25) (layer "B.Cu") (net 4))
 (segment (start 82.55 106.68) (end 76.835 106.68) (width 0.25) (layer "B.Cu") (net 4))
 (segment (start 74.93 45.72) (end 76.835 43.815) (width 1) (layer "B.Cu") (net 4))
 (segment (start 90.17 45.72) (end 90.17 48.26) (width 1) (layer "B.Cu") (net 4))
 (segment (start 74.93 81.915) (end 83.185 73.66) (width 0.25) (layer "B.Cu") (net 4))
 (segment (start 83.185 73.66) (end 83.185 55.245) (width 0.25) (layer "B.Cu") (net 4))
 (segment (start 83.82 105.41) (end 82.55 106.68) (width 0.25) (layer "B.Cu") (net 4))
 (segment (start 83.82 102.7275) (end 83.82 105.41) (width 0.25) (layer "B.Cu") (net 4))
 (segment (start 83.185 55.245) (end 90.17 48.26) (width 0.25) (layer "B.Cu") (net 4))
 (segment (start 129.54 66.04) (end 118.11 66.04) (width 0.25) (layer "B.Cu") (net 23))
 (segment (start 113.665 85.725) (end 110.49 88.9) (width 0.25) (layer "B.Cu") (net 23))
 (segment (start 108.0925 88.9) (end 104.14 84.9475) (width 0.25) (layer "B.Cu") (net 23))
 (segment (start 118.11 66.04) (end 113.665 70.485) (width 0.25) (layer "B.Cu") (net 23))
 (segment (start 110.49 88.9) (end 108.0925 88.9) (width 0.25) (layer "B.Cu") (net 23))
 (segment (start 149.86 91.44) (end 146.608856 91.44) (width 0.25) (layer "B.Cu") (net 23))
 (segment (start 146.608856 91.44) (end 136.525 81.356144) (width 0.25) (layer "B.Cu") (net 23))
 (segment (start 136.525 73.025) (end 129.54 66.04) (width 0.25) (layer "B.Cu") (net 23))
 (segment (start 136.525 81.356144) (end 136.525 73.025) (width 0.25) (layer "B.Cu") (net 23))
 (segment (start 113.665 70.485) (end 113.665 85.725) (width 0.25) (layer "B.Cu") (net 23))
 (segment (start 56.515 104.14) (end 55.245 102.87) (width 0.25) (layer "F.Cu") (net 39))
 (segment (start 55.245 81.915) (end 57.785 79.375) (width 0.25) (layer "F.Cu") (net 39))
 (segment (start 57.785 70.485) (end 53.34 66.04) (width 0.25) (layer "F.Cu") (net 39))
 (segment (start 58.105 104.14) (end 56.515 104.14) (width 0.25) (layer "F.Cu") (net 39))
 (segment (start 55.245 102.87) (end 55.245 81.915) (width 0.25) (layer "F.Cu") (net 39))
 (segment (start 57.785 79.375) (end 57.785 70.485) (width 0.25) (layer "F.Cu") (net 39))
 (segment (start 53.34 66.04) (end 53.34 61.435) (width 0.25) (layer "F.Cu") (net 39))
 (segment (start 74.295 95.885) (end 69.85 100.33) (width 0.25) (layer "F.Cu") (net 17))
 (segment (start 149.86 76.2) (end 145.415 76.2) (width 0.25) (layer "F.Cu") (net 17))
 (segment (start 145.415 76.2) (end 125.73 95.885) (width 0.25) (layer "F.Cu") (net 17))
 (segment (start 69.85 100.33) (end 69.85 104.14) (width 0.25) (layer "F.Cu") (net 17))
 (segment (start 125.73 95.885) (end 74.295 95.885) (width 0.25) (layer "F.Cu") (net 17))
 (segment (start 68.2 100.33) (end 62.865 100.33) (width 0.25) (layer "F.Cu") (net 24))
 (segment (start 62.865 100.33) (end 61.595 99.06) (width 0.25) (layer "F.Cu") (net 24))
 (segment (start 52.705 99.06) (end 48.575 99.06) (width 0.25) (layer "F.Cu") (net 24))
 (via (at 61.595 99.06) (size 0.8) (drill 0.4) (layers "F.Cu" "B.Cu") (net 24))
 (via (at 52.705 99.06) (size 0.8) (drill 0.4) (layers "F.Cu" "B.Cu") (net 24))
 (segment (start 61.595 99.06) (end 52.705 99.06) (width 0.25) (layer "B.Cu") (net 24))
 (segment (start 109.22 109.22) (end 119.38 99.06) (width 0.25) (layer "F.Cu") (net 13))
 (segment (start 106.68 114.14) (end 109.22 114.14) (width 0.25) (layer "F.Cu") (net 13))
 (segment (start 109.22 114.14) (end 109.22 109.22) (width 0.25) (layer "F.Cu") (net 13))
 (via (at 119.38 99.06) (size 0.8) (drill 0.4) (layers "F.Cu" "B.Cu") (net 13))
 (segment (start 124.46 88.9) (end 119.38 93.98) (width 0.25) (layer "B.Cu") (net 13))
 (segment (start 119.38 93.98) (end 119.38 99.06) (width 0.25) (layer "B.Cu") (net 13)))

